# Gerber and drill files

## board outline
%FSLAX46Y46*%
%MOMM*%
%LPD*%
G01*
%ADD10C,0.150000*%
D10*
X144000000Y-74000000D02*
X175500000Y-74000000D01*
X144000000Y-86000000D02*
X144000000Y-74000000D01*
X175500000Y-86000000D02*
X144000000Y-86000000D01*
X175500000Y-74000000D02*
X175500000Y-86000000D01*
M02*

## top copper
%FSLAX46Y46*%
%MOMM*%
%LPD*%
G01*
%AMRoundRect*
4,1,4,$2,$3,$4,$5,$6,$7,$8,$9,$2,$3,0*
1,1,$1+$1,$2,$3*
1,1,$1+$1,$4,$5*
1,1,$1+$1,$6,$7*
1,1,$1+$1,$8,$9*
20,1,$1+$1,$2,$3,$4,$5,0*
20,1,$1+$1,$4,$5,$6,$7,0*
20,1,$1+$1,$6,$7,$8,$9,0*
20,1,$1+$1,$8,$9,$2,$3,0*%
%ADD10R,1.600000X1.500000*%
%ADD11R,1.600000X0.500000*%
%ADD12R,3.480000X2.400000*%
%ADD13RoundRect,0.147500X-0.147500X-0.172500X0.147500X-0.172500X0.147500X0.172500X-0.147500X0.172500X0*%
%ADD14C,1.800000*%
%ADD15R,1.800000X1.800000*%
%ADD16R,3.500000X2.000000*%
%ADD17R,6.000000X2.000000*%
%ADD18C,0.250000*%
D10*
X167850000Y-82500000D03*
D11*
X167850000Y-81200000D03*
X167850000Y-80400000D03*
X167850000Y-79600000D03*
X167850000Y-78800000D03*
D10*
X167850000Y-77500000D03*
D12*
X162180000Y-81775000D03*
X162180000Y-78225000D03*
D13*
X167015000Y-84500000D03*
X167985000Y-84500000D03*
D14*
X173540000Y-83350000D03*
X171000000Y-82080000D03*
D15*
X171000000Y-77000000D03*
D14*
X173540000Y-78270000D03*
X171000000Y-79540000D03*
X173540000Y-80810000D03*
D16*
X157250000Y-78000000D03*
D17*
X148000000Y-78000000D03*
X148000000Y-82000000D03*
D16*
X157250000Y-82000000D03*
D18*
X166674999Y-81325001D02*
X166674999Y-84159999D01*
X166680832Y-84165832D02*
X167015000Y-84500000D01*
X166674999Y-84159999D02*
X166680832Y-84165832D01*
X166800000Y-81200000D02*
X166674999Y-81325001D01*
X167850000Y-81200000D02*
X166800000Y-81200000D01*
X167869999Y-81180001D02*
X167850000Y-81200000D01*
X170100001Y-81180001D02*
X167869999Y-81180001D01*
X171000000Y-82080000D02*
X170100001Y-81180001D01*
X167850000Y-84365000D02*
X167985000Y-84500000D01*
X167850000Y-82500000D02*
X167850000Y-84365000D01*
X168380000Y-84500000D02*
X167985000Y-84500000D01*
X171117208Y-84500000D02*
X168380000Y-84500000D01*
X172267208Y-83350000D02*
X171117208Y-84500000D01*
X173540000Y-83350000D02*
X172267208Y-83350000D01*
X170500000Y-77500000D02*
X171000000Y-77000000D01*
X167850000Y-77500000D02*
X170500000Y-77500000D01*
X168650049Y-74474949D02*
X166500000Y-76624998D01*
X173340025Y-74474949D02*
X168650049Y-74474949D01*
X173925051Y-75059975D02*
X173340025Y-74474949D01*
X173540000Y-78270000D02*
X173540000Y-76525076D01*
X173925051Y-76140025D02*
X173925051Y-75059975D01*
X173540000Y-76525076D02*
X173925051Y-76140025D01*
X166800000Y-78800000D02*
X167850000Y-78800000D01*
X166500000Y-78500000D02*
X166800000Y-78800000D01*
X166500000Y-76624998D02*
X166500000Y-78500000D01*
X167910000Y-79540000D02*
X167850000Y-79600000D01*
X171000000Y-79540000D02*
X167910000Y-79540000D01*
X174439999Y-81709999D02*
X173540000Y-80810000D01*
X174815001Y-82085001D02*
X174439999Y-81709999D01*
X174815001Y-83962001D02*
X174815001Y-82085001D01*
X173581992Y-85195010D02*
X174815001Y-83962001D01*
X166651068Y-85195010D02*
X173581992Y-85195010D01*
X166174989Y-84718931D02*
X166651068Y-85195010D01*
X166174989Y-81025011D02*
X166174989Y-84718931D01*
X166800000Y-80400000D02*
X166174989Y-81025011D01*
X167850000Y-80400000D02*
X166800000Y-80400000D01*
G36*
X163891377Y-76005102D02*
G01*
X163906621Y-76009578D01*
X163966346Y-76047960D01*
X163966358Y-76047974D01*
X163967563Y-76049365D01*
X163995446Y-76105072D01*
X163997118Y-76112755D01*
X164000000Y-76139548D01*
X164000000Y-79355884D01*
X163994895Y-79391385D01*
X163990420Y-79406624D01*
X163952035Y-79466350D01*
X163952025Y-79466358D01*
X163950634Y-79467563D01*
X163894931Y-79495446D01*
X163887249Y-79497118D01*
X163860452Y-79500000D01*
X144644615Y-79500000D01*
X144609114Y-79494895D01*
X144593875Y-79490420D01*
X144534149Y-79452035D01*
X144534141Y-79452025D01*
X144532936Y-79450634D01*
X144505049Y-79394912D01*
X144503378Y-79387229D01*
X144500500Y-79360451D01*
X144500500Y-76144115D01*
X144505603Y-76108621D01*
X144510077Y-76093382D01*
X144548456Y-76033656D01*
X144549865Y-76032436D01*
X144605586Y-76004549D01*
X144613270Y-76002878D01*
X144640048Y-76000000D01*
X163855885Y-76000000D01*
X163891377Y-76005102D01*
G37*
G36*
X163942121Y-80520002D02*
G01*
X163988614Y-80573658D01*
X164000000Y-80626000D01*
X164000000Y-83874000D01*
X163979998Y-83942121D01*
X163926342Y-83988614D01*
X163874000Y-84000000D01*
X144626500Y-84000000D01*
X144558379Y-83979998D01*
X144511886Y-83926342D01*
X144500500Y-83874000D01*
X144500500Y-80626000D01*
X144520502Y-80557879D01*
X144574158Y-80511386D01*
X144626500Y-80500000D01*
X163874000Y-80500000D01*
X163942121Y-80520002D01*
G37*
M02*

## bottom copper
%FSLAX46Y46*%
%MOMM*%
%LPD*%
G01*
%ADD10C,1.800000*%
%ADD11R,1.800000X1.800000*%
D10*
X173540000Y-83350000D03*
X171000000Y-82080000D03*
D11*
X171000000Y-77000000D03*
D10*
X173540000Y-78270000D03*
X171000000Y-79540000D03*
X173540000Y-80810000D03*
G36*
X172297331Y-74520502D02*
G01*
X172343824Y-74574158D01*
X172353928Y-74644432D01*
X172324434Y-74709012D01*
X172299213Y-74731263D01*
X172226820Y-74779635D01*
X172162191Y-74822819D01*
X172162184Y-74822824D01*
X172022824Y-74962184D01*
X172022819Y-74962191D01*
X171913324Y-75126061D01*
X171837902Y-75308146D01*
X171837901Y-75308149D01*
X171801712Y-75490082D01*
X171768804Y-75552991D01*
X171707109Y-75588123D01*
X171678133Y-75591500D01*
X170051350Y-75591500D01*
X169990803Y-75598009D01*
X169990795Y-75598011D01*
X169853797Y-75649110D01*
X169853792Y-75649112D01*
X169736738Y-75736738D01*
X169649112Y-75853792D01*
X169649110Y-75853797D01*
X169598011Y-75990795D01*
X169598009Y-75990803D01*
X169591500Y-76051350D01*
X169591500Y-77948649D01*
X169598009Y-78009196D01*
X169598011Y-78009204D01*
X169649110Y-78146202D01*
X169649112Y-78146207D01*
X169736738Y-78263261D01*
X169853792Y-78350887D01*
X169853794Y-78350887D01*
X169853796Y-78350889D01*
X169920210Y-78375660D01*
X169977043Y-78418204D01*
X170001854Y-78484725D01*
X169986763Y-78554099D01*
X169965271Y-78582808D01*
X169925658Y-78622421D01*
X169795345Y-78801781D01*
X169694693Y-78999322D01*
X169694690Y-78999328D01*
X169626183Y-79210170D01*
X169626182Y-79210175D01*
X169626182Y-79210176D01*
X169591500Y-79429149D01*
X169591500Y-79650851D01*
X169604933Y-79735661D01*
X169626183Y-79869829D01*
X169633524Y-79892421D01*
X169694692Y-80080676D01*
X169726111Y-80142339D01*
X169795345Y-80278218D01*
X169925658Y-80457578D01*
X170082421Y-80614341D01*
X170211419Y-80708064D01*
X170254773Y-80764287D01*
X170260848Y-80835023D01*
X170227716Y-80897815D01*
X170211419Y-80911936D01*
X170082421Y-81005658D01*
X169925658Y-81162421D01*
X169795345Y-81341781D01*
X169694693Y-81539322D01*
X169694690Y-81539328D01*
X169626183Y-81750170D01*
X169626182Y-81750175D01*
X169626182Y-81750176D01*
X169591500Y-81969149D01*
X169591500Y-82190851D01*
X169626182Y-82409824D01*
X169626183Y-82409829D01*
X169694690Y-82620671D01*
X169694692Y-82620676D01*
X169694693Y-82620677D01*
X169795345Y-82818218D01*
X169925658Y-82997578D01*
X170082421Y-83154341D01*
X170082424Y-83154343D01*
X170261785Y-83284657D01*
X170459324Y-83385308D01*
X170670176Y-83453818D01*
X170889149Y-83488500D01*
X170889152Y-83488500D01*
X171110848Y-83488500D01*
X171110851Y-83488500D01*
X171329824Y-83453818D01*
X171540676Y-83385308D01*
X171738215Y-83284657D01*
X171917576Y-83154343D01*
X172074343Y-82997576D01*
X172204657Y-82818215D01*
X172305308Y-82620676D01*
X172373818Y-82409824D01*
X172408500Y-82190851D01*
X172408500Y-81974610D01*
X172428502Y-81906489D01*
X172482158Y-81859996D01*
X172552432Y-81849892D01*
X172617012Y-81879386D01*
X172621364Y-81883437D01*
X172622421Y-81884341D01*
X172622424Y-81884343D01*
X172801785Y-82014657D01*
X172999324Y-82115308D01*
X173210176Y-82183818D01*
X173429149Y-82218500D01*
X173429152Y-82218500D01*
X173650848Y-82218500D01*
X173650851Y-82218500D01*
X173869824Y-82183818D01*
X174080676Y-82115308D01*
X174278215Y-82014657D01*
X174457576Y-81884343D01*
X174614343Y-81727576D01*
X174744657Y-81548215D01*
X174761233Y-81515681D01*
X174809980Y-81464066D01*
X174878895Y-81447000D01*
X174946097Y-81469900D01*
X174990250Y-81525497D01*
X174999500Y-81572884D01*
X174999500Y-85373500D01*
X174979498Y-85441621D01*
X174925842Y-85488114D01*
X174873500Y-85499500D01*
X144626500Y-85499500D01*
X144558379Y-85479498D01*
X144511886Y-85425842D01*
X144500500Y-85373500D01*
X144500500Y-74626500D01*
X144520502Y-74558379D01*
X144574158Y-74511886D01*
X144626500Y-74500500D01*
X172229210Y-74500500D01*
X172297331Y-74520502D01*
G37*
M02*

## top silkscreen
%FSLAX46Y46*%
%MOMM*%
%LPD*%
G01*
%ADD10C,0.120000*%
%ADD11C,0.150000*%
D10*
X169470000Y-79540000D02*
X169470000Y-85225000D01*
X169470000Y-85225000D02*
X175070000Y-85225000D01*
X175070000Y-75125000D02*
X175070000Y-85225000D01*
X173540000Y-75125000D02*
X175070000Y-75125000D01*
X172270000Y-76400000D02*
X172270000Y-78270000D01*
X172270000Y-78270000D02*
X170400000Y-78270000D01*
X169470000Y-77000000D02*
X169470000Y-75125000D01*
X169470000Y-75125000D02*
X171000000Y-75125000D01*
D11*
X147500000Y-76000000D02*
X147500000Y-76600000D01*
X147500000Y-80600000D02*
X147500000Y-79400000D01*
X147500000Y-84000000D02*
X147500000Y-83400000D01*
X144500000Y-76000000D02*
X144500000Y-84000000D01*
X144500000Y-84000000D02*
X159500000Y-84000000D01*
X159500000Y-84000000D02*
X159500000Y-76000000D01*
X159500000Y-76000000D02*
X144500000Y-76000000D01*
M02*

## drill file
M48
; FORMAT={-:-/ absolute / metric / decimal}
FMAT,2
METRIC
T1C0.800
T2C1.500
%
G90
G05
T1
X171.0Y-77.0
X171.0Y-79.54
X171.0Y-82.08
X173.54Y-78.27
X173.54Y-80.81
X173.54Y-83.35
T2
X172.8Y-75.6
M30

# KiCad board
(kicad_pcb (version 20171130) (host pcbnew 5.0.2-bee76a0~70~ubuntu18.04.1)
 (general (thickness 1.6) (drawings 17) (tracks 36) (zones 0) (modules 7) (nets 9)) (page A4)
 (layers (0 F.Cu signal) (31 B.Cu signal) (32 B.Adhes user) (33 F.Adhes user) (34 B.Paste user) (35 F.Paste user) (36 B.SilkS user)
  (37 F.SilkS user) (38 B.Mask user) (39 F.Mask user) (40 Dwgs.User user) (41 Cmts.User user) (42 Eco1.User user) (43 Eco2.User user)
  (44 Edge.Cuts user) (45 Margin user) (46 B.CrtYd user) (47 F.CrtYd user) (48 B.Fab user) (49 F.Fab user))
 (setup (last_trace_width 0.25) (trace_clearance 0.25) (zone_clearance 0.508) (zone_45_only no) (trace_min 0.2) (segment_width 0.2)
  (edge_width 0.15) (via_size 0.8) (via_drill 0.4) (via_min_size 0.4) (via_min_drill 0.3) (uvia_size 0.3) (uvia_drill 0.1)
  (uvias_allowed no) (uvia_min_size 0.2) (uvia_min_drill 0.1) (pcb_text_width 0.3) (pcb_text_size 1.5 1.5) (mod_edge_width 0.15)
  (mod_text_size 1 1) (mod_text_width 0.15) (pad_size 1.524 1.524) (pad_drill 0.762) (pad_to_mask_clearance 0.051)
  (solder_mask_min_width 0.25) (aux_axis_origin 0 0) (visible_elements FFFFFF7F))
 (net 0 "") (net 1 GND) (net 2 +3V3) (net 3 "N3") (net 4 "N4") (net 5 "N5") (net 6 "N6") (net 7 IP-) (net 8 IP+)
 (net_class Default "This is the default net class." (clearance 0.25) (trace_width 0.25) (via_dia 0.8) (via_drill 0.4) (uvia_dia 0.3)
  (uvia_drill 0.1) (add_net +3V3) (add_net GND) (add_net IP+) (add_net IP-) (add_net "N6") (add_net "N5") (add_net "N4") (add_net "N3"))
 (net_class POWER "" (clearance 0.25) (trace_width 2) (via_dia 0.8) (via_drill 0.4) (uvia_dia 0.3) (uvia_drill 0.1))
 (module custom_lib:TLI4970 (layer F.Cu) (at 164.5 80 90)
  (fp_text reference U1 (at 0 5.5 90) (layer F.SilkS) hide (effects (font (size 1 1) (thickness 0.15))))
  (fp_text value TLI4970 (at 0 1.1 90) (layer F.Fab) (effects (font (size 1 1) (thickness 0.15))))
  (pad 1 smd rect (at -2.5 3.35 270) (size 1.5 1.6) (layers F.Cu F.Paste F.Mask) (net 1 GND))
  (pad 2 smd rect (at -1.2 3.35 270) (size 0.5 1.6) (layers F.Cu F.Paste F.Mask) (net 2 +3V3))
  (pad 3 smd rect (at -0.4 3.35 270) (size 0.5 1.6) (layers F.Cu F.Paste F.Mask) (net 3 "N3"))
  (pad 4 smd rect (at 0.4 3.35 270) (size 0.5 1.6) (layers F.Cu F.Paste F.Mask) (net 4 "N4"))
  (pad 5 smd rect (at 1.2 3.35 270) (size 0.5 1.6) (layers F.Cu F.Paste F.Mask) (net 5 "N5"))
  (pad 6 smd rect (at 2.5 3.35 270) (size 1.5 1.6) (layers F.Cu F.Paste F.Mask) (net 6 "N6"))
  (pad 8 smd rect (at -1.775 -2.32 270) (size 2.4 3.48) (layers F.Cu F.Paste F.Mask) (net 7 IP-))
  (pad 7 smd rect (at 1.775 -2.32 270) (size 2.4 3.48) (layers F.Cu F.Paste F.Mask) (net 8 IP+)))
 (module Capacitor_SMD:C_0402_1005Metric (layer F.Cu) (at 167.5 84.5)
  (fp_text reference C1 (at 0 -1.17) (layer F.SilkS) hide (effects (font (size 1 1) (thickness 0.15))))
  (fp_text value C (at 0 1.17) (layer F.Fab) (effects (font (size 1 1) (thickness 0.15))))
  (pad 1 smd roundrect (at -0.485 0) (size 0.59 0.64) (layers F.Cu F.Paste F.Mask) (roundrect_rratio 0.25) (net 2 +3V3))
  (pad 2 smd roundrect (at 0.485 0) (size 0.59 0.64) (layers F.Cu F.Paste F.Mask) (roundrect_rratio 0.25) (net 1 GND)))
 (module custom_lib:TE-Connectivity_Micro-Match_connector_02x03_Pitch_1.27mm (layer F.Cu) (at 171 77)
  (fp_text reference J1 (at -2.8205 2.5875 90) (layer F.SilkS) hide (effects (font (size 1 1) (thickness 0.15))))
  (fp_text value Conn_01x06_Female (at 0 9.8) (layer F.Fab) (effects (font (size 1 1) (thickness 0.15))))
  (fp_line (start -1.53 2.54) (end -1.53 8.225) (layer F.SilkS) (width 0.12))
  (fp_line (start -1.53 8.225) (end 4.07 8.225) (layer F.SilkS) (width 0.12))
  (fp_line (start 4.07 -1.875) (end 4.07 8.225) (layer F.SilkS) (width 0.12))
  (fp_line (start 2.54 -1.875) (end 4.07 -1.875) (layer F.SilkS) (width 0.12))
  (fp_line (start 1.27 -0.6) (end 1.27 1.27) (layer F.SilkS) (width 0.12))
  (fp_line (start 1.27 1.27) (end -0.6 1.27) (layer F.SilkS) (width 0.12))
  (fp_line (start -1.53 0) (end -1.53 -1.875) (layer F.SilkS) (width 0.12))
  (fp_line (start -1.53 -1.875) (end 0 -1.875) (layer F.SilkS) (width 0.12))
  (pad 6 thru_hole circle (at 2.54 6.35) (size 1.8 1.8) (drill 0.8001) (layers *.Cu *.Mask) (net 1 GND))
  (pad 5 thru_hole circle (at 0 5.08) (size 1.8 1.8) (drill 0.8001) (layers *.Cu *.Mask) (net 2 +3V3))
  (pad 1 thru_hole rect (at 0 0) (size 1.8 1.8) (drill 0.8001) (layers *.Cu *.Mask) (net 6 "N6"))
  (pad 2 thru_hole circle (at 2.54 1.27) (size 1.8 1.8) (drill 0.8001) (layers *.Cu *.Mask) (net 5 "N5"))
  (pad 3 thru_hole circle (at 0 2.54) (size 1.8 1.8) (drill 0.8001) (layers *.Cu *.Mask) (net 4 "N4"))
  (pad 4 thru_hole circle (at 2.54 3.81) (size 1.8 1.8) (drill 0.8001) (layers *.Cu *.Mask) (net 3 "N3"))
  (pad "" np_thru_hole circle (at 1.8 -1.4) (size 1.5001 1.5001) (drill 1.5001) (layers *.Cu *.Mask)))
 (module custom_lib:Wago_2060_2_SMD (layer F.Cu) (at 152 80 90)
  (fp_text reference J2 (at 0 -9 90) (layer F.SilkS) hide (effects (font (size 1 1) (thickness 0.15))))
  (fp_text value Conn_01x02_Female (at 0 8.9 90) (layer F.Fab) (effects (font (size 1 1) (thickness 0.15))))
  (fp_line (start 4 -4.5) (end 3.4 -4.5) (layer F.SilkS) (width 0.15))
  (fp_line (start -0.6 -4.5) (end 0.6 -4.5) (layer F.SilkS) (width 0.15))
  (fp_line (start -4 -4.5) (end -3.4 -4.5) (layer F.SilkS) (width 0.15))
  (fp_line (start 4 -7.5) (end -4 -7.5) (layer F.SilkS) (width 0.15))
  (fp_line (start -4 -7.5) (end -4 7.5) (layer F.SilkS) (width 0.15))
  (fp_line (start -4 7.5) (end 4 7.5) (layer F.SilkS) (width 0.15))
  (fp_line (start 4 7.5) (end 4 -7.5) (layer F.SilkS) (width 0.15))
  (pad 2 smd rect (at 2 5.25 90) (size 2 3.5) (layers F.Cu F.Paste F.Mask) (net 8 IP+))
  (pad 2 smd rect (at 2 -4 90) (size 2 6) (layers F.Cu F.Paste F.Mask) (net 8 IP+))
  (pad 1 smd rect (at -2 -4 90) (size 2 6) (layers F.Cu F.Paste F.Mask) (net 7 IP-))
  (pad 1 smd rect (at -2 5.25 90) (size 2 3.5) (layers F.Cu F.Paste F.Mask) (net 7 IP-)))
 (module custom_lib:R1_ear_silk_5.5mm (layer B.Cu) (at 148.235873 77.900252 180)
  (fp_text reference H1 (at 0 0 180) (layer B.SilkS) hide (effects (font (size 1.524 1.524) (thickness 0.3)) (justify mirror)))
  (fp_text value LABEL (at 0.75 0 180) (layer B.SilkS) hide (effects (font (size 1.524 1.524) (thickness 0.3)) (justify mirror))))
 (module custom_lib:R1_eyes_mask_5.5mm (layer B.Cu) (at 148.245873 77.850252 180)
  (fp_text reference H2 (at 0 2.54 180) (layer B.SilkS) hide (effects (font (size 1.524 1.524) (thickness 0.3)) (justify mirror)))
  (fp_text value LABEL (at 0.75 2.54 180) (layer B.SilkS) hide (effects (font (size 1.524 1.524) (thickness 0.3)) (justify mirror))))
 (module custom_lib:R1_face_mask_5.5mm (layer B.Cu) (at 148.23303 77.898191 180)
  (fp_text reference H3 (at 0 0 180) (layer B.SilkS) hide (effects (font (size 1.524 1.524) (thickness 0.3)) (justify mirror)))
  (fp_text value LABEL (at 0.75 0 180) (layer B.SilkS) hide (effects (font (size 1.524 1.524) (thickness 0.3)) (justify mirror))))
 (gr_line (start 144 74) (end 175.5 74) (layer Edge.Cuts) (width 0.15))
 (gr_line (start 144 86) (end 144 74) (layer Edge.Cuts) (width 0.15))
 (gr_line (start 175.5 86) (end 144 86) (layer Edge.Cuts) (width 0.15))
 (gr_line (start 175.5 74) (end 175.5 86) (layer Edge.Cuts) (width 0.15))
 (segment (start 166.674999 81.325001) (end 166.674999 84.159999) (width 0.25) (layer F.Cu) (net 2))
 (segment (start 166.680832 84.165832) (end 167.015 84.5) (width 0.25) (layer F.Cu) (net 2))
 (segment (start 166.674999 84.159999) (end 166.680832 84.165832) (width 0.25) (layer F.Cu) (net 2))
 (segment (start 166.8 81.2) (end 166.674999 81.325001) (width 0.25) (layer F.Cu) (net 2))
 (segment (start 167.85 81.2) (end 166.8 81.2) (width 0.25) (layer F.Cu) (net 2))
 (segment (start 167.869999 81.180001) (end 167.85 81.2) (width 0.25) (layer F.Cu) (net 2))
 (segment (start 170.100001 81.180001) (end 167.869999 81.180001) (width 0.25) (layer F.Cu) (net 2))
 (segment (start 171 82.08) (end 170.100001 81.180001) (width 0.25) (layer F.Cu) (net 2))
 (segment (start 167.85 84.365) (end 167.985 84.5) (width 0.25) (layer F.Cu) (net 1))
 (segment (start 167.85 82.5) (end 167.85 84.365) (width 0.25) (layer F.Cu) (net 1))
 (segment (start 168.38 84.5) (end 167.985 84.5) (width 0.25) (layer F.Cu) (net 1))
 (segment (start 171.117208 84.5) (end 168.38 84.5) (width 0.25) (layer F.Cu) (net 1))
 (segment (start 172.267208 83.35) (end 171.117208 84.5) (width 0.25) (layer F.Cu) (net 1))
 (segment (start 173.54 83.35) (end 172.267208 83.35) (width 0.25) (layer F.Cu) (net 1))
 (segment (start 170.5 77.5) (end 171 77) (width 0.25) (layer F.Cu) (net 6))
 (segment (start 167.85 77.5) (end 170.5 77.5) (width 0.25) (layer F.Cu) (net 6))
 (segment (start 168.650049 74.474949) (end 166.5 76.624998) (width 0.25) (layer F.Cu) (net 5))
 (segment (start 173.340025 74.474949) (end 168.650049 74.474949) (width 0.25) (layer F.Cu) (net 5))
 (segment (start 173.925051 75.059975) (end 173.340025 74.474949) (width 0.25) (layer F.Cu) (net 5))
 (segment (start 173.54 78.27) (end 173.54 76.525076) (width 0.25) (layer F.Cu) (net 5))
 (segment (start 173.925051 76.140025) (end 173.925051 75.059975) (width 0.25) (layer F.Cu) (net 5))
 (segment (start 173.54 76.525076) (end 173.925051 76.140025) (width 0.25) (layer F.Cu) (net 5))
 (segment (start 166.8 78.8) (end 167.85 78.8) (width 0.25) (layer F.Cu) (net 5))
 (segment (start 166.5 78.5) (end 166.8 78.8) (width 0.25) (layer F.Cu) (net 5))
 (segment (start 166.5 76.624998) (end 166.5 78.5) (width 0.25) (layer F.Cu) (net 5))
 (segment (start 167.91 79.54) (end 167.85 79.6) (width 0.25) (layer F.Cu) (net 4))
 (segment (start 171 79.54) (end 167.91 79.54) (width 0.25) (layer F.Cu) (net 4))
 (segment (start 174.439999 81.709999) (end 173.54 80.81) (width 0.25) (layer F.Cu) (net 3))
 (segment (start 174.815001 82.085001) (end 174.439999 81.709999) (width 0.25) (layer F.Cu) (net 3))
 (segment (start 174.815001 83.962001) (end 174.815001 82.085001) (width 0.25) (layer F.Cu) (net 3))
 (segment (start 173.581992 85.19501) (end 174.815001 83.962001) (width 0.25) (layer F.Cu) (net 3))
 (segment (start 166.651068 85.19501) (end 173.581992 85.19501) (width 0.25) (layer F.Cu) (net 3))
 (segment (start 166.174989 84.718931) (end 166.651068 85.19501) (width 0.25) (layer F.Cu) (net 3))
 (segment (start 166.174989 81.025011) (end 166.174989 84.718931) (width 0.25) (layer F.Cu) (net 3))
 (segment (start 166.8 80.4) (end 166.174989 81.025011) (width 0.25) (layer F.Cu) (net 3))
 (segment (start 167.85 80.4) (end 166.8 80.4) (width 0.25) (layer F.Cu) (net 3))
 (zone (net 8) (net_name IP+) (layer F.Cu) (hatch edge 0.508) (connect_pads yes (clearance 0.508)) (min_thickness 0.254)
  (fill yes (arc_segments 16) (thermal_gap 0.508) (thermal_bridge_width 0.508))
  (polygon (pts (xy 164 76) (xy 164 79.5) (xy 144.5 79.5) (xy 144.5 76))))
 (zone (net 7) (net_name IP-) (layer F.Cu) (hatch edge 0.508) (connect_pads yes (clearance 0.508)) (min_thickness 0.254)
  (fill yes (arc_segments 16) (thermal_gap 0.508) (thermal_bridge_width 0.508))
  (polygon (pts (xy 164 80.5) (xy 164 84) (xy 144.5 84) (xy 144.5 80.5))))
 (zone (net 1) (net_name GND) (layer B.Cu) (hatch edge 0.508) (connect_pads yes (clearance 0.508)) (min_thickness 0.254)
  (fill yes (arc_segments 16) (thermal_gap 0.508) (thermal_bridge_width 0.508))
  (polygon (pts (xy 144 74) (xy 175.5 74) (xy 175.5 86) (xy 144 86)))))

